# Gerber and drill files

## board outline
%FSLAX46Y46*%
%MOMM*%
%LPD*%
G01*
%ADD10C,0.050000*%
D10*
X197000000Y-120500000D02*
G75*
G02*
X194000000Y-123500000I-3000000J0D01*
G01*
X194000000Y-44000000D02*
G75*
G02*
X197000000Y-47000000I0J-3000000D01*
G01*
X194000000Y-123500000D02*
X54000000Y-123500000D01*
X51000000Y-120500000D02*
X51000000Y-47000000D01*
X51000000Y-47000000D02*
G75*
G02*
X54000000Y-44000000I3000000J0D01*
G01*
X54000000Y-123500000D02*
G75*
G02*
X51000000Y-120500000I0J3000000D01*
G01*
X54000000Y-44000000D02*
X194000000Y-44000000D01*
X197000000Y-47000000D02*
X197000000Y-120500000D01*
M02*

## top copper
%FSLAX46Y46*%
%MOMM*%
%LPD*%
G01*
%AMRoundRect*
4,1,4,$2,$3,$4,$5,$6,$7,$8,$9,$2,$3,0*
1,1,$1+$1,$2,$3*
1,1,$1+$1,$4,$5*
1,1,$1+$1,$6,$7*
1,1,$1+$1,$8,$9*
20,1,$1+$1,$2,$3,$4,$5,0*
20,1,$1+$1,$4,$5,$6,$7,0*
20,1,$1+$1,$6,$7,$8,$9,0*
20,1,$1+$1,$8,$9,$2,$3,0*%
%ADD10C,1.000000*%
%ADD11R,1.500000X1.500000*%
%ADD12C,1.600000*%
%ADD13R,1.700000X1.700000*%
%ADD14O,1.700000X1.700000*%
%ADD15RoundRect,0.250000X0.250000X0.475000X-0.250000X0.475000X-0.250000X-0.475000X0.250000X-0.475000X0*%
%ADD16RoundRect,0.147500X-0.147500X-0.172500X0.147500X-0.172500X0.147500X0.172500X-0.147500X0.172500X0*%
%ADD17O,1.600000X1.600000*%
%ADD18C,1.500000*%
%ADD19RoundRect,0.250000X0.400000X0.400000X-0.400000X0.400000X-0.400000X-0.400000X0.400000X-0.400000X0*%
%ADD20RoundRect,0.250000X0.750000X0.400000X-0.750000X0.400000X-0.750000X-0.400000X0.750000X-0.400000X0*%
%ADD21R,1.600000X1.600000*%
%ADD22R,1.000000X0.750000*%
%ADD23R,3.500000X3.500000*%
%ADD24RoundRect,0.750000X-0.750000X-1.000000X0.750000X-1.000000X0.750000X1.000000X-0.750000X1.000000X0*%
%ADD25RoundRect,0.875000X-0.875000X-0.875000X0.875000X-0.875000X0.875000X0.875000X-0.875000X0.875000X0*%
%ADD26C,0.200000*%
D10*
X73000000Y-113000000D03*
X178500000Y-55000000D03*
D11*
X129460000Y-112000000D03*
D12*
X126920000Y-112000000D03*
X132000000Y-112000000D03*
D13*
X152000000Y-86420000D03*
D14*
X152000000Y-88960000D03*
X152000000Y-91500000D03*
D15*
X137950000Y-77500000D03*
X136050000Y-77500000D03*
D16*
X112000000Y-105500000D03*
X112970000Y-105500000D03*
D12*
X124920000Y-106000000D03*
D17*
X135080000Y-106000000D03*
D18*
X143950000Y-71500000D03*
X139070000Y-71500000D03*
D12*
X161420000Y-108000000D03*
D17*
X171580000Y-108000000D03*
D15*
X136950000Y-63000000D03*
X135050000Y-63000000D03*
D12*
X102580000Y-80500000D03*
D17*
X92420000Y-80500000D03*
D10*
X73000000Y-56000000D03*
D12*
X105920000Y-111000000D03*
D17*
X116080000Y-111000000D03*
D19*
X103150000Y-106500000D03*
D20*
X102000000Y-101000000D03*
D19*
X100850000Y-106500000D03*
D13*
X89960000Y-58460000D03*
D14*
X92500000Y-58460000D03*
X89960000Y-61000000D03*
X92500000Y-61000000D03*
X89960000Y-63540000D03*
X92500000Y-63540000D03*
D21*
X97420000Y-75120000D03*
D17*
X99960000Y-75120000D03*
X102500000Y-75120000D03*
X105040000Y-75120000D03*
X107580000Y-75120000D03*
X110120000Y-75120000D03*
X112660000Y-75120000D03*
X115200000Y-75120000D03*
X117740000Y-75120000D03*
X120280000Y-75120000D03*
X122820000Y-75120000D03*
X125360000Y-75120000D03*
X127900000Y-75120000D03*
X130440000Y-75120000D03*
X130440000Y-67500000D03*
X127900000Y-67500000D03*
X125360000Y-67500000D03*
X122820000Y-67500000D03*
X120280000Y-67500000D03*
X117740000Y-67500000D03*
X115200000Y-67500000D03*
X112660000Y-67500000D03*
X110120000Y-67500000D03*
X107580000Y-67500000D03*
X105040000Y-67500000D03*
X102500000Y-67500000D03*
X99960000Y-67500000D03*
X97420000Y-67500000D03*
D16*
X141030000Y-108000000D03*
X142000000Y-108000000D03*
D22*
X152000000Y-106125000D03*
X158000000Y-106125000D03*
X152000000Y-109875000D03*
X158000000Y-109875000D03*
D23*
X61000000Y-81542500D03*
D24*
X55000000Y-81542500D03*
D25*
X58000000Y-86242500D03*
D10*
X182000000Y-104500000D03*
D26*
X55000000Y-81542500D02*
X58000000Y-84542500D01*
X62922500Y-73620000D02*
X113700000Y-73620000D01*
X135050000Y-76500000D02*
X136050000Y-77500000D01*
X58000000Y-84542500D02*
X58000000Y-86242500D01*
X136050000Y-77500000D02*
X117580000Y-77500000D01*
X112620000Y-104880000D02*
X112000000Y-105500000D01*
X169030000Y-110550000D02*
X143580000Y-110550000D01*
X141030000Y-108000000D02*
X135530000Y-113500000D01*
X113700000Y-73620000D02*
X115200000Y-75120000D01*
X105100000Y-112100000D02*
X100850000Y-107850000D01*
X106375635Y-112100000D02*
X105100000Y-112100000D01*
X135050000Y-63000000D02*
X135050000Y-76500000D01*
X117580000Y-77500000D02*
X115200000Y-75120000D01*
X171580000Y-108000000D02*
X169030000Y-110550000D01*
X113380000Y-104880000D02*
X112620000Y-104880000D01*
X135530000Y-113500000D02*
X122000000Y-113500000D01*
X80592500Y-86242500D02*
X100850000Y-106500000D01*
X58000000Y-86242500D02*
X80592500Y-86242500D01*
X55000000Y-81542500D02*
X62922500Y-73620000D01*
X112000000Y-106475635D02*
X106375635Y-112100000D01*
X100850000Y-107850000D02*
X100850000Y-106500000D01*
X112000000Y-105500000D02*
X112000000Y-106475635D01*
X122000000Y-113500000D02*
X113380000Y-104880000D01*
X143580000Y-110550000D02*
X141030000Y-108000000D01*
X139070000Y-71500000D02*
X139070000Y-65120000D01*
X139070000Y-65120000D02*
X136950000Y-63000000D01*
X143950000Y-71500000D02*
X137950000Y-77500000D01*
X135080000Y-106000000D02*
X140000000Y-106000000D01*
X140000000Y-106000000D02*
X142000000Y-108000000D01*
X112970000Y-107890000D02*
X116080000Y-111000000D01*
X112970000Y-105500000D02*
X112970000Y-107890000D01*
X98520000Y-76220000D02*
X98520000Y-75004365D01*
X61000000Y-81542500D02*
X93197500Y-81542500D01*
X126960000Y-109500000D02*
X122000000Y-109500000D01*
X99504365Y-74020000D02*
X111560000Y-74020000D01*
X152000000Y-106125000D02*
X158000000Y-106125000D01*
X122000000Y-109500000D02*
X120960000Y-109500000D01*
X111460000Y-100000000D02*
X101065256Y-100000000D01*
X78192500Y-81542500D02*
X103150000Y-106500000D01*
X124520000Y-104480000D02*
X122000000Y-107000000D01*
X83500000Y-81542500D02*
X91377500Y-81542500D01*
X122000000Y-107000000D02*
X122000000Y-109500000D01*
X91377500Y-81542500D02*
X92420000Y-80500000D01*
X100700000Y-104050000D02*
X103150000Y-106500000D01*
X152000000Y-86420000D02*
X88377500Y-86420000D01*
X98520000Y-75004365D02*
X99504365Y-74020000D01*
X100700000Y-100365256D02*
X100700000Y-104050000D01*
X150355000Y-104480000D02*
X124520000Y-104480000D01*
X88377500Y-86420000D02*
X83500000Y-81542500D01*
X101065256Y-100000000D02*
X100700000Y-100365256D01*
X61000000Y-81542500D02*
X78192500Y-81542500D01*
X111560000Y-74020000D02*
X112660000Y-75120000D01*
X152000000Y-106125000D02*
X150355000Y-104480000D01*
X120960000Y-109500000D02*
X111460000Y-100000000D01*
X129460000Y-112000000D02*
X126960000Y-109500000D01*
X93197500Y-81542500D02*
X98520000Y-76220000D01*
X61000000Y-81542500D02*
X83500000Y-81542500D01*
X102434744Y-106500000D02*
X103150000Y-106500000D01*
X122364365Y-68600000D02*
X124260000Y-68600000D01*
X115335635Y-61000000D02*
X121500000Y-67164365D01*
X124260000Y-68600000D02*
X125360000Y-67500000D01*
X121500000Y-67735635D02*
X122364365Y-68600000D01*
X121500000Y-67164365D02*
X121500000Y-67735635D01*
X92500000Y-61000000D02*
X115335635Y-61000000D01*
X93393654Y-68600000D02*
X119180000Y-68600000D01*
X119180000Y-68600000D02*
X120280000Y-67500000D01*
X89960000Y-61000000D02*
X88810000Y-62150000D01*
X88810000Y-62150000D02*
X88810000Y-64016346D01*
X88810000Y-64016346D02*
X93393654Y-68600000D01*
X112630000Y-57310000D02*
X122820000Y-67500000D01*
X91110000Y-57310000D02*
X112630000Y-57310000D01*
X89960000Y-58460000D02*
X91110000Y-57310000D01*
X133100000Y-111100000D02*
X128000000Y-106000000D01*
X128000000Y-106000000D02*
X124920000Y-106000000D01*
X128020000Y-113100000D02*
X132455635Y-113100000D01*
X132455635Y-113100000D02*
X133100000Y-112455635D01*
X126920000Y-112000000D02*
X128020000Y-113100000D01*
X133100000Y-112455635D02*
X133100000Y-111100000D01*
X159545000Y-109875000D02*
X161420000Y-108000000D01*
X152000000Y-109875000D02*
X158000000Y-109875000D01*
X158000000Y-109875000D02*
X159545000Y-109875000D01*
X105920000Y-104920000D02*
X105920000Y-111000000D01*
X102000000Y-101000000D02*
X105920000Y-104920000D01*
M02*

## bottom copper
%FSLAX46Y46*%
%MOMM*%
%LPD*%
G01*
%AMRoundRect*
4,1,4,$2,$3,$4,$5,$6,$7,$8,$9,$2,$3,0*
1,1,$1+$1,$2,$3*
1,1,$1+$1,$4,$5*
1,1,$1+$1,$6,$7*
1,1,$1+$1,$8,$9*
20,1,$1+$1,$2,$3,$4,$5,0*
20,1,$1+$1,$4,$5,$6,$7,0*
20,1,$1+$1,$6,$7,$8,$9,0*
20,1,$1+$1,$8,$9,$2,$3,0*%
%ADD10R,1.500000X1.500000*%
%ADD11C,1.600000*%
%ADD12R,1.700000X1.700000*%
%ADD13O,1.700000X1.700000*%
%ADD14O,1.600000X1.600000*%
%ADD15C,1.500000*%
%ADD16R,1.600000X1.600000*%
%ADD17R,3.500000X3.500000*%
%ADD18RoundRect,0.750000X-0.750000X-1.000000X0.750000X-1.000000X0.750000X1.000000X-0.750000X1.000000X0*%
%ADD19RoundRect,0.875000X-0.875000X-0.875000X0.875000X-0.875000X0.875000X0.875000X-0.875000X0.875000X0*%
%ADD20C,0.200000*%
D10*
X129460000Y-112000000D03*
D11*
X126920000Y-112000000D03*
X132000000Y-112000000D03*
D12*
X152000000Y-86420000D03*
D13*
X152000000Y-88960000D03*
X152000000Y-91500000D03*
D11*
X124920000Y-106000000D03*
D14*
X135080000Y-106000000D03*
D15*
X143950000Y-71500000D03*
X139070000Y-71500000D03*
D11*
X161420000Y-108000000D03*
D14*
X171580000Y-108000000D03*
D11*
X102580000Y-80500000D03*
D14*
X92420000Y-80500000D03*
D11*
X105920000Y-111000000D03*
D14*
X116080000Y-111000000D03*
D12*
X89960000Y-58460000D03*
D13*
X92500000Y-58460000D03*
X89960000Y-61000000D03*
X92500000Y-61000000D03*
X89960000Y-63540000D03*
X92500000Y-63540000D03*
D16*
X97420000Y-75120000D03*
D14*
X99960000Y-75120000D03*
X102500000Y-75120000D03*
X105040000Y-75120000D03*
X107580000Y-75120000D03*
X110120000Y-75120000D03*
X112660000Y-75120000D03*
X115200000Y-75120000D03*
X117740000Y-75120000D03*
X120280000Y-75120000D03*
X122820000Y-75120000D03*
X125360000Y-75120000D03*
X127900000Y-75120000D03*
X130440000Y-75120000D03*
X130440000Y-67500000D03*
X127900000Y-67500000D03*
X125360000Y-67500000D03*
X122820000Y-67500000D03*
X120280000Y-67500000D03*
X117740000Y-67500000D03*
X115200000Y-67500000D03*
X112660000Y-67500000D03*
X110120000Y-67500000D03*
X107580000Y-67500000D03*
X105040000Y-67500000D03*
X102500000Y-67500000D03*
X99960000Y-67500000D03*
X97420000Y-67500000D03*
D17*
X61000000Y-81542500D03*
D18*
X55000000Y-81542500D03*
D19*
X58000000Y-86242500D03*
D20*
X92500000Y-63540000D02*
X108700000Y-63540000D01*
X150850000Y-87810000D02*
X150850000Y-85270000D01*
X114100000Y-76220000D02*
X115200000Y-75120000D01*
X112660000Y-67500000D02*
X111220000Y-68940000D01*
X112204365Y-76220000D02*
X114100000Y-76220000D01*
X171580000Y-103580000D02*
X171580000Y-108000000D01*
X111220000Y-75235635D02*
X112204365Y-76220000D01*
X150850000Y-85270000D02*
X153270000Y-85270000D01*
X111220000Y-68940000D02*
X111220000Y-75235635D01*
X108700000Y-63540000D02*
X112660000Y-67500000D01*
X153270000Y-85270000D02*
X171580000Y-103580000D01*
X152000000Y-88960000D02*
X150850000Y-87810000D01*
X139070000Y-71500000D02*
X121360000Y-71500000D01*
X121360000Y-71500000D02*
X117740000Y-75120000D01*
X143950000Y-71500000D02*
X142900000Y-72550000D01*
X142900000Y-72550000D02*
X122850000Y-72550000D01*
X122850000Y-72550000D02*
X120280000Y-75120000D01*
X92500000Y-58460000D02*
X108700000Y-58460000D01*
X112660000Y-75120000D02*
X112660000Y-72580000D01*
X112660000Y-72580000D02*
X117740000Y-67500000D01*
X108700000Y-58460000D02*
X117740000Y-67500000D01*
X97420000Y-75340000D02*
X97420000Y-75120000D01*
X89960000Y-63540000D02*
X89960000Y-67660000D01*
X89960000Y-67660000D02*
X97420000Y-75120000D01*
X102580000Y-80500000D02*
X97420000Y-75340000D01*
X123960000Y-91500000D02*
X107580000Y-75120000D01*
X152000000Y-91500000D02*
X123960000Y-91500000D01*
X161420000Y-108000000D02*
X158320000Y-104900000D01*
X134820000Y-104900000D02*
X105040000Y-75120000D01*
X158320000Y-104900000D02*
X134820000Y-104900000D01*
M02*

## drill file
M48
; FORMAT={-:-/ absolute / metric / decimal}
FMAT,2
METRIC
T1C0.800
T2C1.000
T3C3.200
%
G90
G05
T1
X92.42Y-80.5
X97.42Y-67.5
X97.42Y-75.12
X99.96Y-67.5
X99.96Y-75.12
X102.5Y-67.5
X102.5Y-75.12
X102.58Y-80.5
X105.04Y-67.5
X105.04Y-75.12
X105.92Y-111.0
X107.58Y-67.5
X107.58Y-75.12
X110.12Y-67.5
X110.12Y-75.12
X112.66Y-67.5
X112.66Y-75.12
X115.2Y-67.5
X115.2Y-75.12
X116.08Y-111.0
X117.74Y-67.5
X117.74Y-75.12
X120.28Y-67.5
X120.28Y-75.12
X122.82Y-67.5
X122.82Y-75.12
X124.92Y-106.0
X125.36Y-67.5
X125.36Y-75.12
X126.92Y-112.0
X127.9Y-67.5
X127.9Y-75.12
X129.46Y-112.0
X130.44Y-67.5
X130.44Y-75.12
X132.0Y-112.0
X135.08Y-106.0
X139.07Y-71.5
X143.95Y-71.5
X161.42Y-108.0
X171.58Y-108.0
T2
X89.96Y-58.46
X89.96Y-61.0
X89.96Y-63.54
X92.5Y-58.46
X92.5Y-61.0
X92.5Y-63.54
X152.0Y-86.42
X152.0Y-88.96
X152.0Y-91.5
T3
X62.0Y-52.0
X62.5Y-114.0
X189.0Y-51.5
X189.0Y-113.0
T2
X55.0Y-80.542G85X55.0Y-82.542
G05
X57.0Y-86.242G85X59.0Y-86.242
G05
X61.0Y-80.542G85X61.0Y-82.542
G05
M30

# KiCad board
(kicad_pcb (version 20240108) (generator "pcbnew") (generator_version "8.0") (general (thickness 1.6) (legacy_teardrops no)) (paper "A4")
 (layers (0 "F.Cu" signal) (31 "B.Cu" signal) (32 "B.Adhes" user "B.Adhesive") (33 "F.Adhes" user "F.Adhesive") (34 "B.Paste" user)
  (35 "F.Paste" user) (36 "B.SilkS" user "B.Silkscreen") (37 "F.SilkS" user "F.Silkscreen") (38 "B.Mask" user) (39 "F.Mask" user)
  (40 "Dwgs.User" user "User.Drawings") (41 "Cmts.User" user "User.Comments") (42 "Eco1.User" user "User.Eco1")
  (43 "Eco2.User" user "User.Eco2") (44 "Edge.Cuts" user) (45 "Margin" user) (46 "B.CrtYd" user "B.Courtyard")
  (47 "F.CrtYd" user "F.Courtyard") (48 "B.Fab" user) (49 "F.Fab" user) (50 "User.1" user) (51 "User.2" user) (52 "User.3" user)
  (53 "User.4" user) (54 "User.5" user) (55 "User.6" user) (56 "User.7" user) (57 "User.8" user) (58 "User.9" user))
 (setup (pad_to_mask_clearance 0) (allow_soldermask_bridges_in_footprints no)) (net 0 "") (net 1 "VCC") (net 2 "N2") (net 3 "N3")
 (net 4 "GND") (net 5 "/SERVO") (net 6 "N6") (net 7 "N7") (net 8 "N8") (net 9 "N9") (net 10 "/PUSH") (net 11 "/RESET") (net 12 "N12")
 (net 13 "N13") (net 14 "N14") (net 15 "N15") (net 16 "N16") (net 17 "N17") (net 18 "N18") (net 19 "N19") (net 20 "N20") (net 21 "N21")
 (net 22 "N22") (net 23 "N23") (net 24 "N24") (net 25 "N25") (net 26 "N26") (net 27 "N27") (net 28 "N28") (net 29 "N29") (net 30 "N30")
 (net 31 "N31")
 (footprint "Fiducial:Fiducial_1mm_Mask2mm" (layer "F.Cu") (at 73 113)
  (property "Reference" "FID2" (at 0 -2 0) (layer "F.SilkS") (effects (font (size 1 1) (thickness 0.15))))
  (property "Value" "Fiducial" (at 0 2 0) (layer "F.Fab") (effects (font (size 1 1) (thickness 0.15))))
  (pad "" smd circle (at 0 0) (size 1 1) (layers "F.Cu" "F.Mask") (solder_mask_margin 0.5) (clearance 0.5)))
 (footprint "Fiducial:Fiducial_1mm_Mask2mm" (layer "F.Cu") (at 178.5 55)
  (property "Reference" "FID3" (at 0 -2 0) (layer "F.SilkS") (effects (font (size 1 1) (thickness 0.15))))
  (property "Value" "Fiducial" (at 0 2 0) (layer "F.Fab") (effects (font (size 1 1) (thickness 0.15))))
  (pad "" smd circle (at 0 0) (size 1 1) (layers "F.Cu" "F.Mask") (solder_mask_margin 0.5) (clearance 0.5)))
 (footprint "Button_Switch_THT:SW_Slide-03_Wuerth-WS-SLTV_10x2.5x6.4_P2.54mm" (layer "F.Cu") (at 129.46 112)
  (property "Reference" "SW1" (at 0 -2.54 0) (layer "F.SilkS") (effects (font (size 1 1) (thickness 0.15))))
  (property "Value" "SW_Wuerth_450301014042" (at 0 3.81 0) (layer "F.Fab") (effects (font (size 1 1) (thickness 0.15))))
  (pad "1" thru_hole rect (at 0 0) (size 1.5 1.5) (drill 0.8) (layers "*.Cu" "*.Mask") (remove_unused_layers no) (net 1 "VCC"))
  (pad "2" thru_hole circle (at -2.54 0) (size 1.6 1.6) (drill 0.8) (layers "*.Cu" "*.Mask") (remove_unused_layers no) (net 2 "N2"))
  (pad "3" thru_hole circle (at 2.54 0) (size 1.6 1.6) (drill 0.8) (layers "*.Cu" "*.Mask") (remove_unused_layers no) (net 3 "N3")))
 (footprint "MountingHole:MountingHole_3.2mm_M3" (layer "F.Cu") (at 62.5 114)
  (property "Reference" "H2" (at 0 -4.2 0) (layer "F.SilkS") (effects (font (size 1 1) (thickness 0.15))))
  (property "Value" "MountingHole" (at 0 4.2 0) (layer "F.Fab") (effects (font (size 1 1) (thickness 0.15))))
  (pad "" np_thru_hole circle (at 0 0) (size 3.2 3.2) (drill 3.2) (layers "*.Cu" "*.Mask")))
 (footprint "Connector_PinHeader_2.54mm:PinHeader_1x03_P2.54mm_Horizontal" (layer "F.Cu") (at 152 86.42)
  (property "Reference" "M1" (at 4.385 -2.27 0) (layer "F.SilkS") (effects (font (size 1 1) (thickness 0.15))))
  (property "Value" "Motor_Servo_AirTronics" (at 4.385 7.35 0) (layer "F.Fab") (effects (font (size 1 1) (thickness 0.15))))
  (pad "1" thru_hole rect (at 0 0) (size 1.7 1.7) (drill 1) (layers "*.Cu" "*.Mask") (remove_unused_layers no) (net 1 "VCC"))
  (pad "2" thru_hole oval (at 0 2.54) (size 1.7 1.7) (drill 1) (layers "*.Cu" "*.Mask") (remove_unused_layers no) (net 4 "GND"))
  (pad "3" thru_hole oval (at 0 5.08) (size 1.7 1.7) (drill 1) (layers "*.Cu" "*.Mask") (remove_unused_layers no) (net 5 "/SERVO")))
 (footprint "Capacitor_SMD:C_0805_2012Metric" (layer "F.Cu") (at 137 77.5 180)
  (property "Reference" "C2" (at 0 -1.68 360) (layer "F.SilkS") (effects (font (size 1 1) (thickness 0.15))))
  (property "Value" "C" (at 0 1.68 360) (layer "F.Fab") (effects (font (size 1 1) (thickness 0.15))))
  (pad "1" smd roundrect (at -0.95 0 180) (size 1 1.45) (layers "F.Cu" "F.Paste" "F.Mask") (roundrect_rratio 0.25) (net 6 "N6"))
  (pad "2" smd roundrect (at 0.95 0 180) (size 1 1.45) (layers "F.Cu" "F.Paste" "F.Mask") (roundrect_rratio 0.25) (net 4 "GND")))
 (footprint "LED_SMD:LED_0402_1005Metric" (layer "F.Cu") (at 112.485 105.5)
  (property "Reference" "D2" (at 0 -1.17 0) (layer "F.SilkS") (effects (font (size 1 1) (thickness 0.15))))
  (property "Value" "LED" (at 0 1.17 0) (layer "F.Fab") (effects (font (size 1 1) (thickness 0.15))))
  (pad "1" smd roundrect (at -0.485 0) (size 0.59 0.64) (layers "F.Cu" "F.Paste" "F.Mask") (roundrect_rratio 0.25) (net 4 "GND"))
  (pad "2" smd roundrect (at 0.485 0) (size 0.59 0.64) (layers "F.Cu" "F.Paste" "F.Mask") (roundrect_rratio 0.25) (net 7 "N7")))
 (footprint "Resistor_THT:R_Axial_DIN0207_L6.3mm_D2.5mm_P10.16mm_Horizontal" (layer "F.Cu") (at 124.92 106)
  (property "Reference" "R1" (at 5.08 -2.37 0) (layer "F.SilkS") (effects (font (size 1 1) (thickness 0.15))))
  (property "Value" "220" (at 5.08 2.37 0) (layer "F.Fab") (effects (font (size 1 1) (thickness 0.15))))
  (pad "1" thru_hole circle (at 0 0) (size 1.6 1.6) (drill 0.8) (layers "*.Cu" "*.Mask") (remove_unused_layers no) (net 2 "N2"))
  (pad "2" thru_hole oval (at 10.16 0) (size 1.6 1.6) (drill 0.8) (layers "*.Cu" "*.Mask") (remove_unused_layers no) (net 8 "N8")))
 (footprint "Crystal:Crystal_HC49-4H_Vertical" (layer "F.Cu") (at 143.95 71.5 180)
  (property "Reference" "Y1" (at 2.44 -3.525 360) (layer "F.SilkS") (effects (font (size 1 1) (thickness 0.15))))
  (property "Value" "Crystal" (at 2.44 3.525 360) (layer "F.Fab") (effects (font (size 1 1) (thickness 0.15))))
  (pad "1" thru_hole circle (at 0 0 180) (size 1.5 1.5) (drill 0.8) (layers "*.Cu" "*.Mask") (remove_unused_layers no) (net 6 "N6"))
  (pad "2" thru_hole circle (at 4.88 0 180) (size 1.5 1.5) (drill 0.8) (layers "*.Cu" "*.Mask") (remove_unused_layers no) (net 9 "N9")))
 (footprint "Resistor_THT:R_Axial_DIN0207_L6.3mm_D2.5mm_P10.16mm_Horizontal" (layer "F.Cu") (at 161.42 108)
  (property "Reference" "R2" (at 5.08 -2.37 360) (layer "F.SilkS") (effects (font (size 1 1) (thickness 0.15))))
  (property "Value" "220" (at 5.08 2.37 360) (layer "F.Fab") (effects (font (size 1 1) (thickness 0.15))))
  (pad "1" thru_hole circle (at 0 0) (size 1.6 1.6) (drill 0.8) (layers "*.Cu" "*.Mask") (remove_unused_layers no) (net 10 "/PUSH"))
  (pad "2" thru_hole oval (at 10.16 0) (size 1.6 1.6) (drill 0.8) (layers "*.Cu" "*.Mask") (remove_unused_layers no) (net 4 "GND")))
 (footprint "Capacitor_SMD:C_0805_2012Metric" (layer "F.Cu") (at 136 63 180)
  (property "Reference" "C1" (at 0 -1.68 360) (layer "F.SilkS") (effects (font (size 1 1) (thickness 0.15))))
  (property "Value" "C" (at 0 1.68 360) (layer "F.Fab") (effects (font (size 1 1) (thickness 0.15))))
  (pad "1" smd roundrect (at -0.95 0 180) (size 1 1.45) (layers "F.Cu" "F.Paste" "F.Mask") (roundrect_rratio 0.25) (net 9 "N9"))
  (pad "2" smd roundrect (at 0.95 0 180) (size 1 1.45) (layers "F.Cu" "F.Paste" "F.Mask") (roundrect_rratio 0.25) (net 4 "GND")))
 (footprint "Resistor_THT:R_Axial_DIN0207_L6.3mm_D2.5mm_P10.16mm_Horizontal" (layer "F.Cu") (at 102.58 80.5 180)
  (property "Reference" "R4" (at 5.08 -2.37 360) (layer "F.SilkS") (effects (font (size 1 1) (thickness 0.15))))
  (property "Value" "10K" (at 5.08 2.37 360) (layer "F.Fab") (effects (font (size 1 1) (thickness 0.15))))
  (pad "1" thru_hole circle (at 0 0 180) (size 1.6 1.6) (drill 0.8) (layers "*.Cu" "*.Mask") (remove_unused_layers no) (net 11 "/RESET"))
  (pad "2" thru_hole oval (at 10.16 0 180) (size 1.6 1.6) (drill 0.8) (layers "*.Cu" "*.Mask") (remove_unused_layers no) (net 1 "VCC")))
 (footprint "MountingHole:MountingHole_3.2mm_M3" (layer "F.Cu") (at 189 51.5)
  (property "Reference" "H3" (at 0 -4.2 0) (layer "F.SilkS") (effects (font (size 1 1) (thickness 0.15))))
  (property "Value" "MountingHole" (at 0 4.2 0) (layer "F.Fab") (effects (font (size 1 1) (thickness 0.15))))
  (pad "" np_thru_hole circle (at 0 0) (size 3.2 3.2) (drill 3.2) (layers "*.Cu" "*.Mask")))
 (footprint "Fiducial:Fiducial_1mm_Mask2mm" (layer "F.Cu") (at 73 56)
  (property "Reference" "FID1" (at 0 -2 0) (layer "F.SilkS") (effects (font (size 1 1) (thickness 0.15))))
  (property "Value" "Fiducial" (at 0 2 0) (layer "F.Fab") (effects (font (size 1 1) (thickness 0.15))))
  (pad "" smd circle (at 0 0) (size 1 1) (layers "F.Cu" "F.Mask") (solder_mask_margin 0.5) (clearance 0.5)))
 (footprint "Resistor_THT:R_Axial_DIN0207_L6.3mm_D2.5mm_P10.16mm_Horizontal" (layer "F.Cu") (at 105.92 111)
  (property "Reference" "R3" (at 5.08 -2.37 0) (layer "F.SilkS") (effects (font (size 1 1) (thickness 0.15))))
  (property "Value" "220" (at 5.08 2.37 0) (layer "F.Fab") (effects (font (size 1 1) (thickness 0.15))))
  (pad "1" thru_hole circle (at 0 0) (size 1.6 1.6) (drill 0.8) (layers "*.Cu" "*.Mask") (remove_unused_layers no) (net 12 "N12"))
  (pad "2" thru_hole oval (at 10.16 0) (size 1.6 1.6) (drill 0.8) (layers "*.Cu" "*.Mask") (remove_unused_layers no) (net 7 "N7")))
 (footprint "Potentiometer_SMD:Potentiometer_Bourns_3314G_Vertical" (layer "F.Cu") (at 102 103.75 180)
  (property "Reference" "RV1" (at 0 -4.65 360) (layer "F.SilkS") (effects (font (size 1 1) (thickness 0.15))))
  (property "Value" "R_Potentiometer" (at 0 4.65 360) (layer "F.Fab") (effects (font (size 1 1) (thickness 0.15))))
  (pad "1" smd roundrect (at -1.15 -2.75 180) (size 1.3 1.3) (layers "F.Cu" "F.Paste" "F.Mask") (roundrect_rratio 0.1923076923)
   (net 1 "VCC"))
  (pad "2" smd roundrect (at 0 2.75 180) (size 2 1.3) (layers "F.Cu" "F.Paste" "F.Mask") (roundrect_rratio 0.1923076923) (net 12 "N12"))
  (pad "3" smd roundrect (at 1.15 -2.75 180) (size 1.3 1.3) (layers "F.Cu" "F.Paste" "F.Mask") (roundrect_rratio 0.1923076923) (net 4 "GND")))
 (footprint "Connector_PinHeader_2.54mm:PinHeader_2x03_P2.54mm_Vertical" (layer "F.Cu") (at 89.96 58.46)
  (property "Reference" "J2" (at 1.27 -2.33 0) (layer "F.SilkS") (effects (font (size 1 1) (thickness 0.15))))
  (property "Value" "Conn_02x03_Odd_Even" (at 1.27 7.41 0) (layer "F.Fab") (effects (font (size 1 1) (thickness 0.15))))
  (pad "1" thru_hole rect (at 0 0) (size 1.7 1.7) (drill 1) (layers "*.Cu" "*.Mask") (remove_unused_layers no) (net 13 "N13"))
  (pad "2" thru_hole oval (at 2.54 0) (size 1.7 1.7) (drill 1) (layers "*.Cu" "*.Mask") (remove_unused_layers no) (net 1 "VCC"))
  (pad "3" thru_hole oval (at 0 2.54) (size 1.7 1.7) (drill 1) (layers "*.Cu" "*.Mask") (remove_unused_layers no) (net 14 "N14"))
  (pad "4" thru_hole oval (at 2.54 2.54) (size 1.7 1.7) (drill 1) (layers "*.Cu" "*.Mask") (remove_unused_layers no) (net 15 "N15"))
  (pad "5" thru_hole oval (at 0 5.08) (size 1.7 1.7) (drill 1) (layers "*.Cu" "*.Mask") (remove_unused_layers no) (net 11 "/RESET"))
  (pad "6" thru_hole oval (at 2.54 5.08) (size 1.7 1.7) (drill 1) (layers "*.Cu" "*.Mask") (remove_unused_layers no) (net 4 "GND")))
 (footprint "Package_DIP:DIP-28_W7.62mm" (layer "F.Cu") (at 97.42 75.12 90)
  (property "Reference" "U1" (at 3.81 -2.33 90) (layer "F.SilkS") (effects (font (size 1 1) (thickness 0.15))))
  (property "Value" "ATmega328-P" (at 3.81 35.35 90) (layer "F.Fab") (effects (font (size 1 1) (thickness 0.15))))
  (pad "1" thru_hole rect (at 0 0 90) (size 1.6 1.6) (drill 0.8) (layers "*.Cu" "*.Mask") (remove_unused_layers no) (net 11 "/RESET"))
  (pad "2" thru_hole oval (at 0 2.54 90) (size 1.6 1.6) (drill 0.8) (layers "*.Cu" "*.Mask") (remove_unused_layers no) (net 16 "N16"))
  (pad "3" thru_hole oval (at 0 5.08 90) (size 1.6 1.6) (drill 0.8) (layers "*.Cu" "*.Mask") (remove_unused_layers no) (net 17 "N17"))
  (pad "4" thru_hole oval (at 0 7.62 90) (size 1.6 1.6) (drill 0.8) (layers "*.Cu" "*.Mask") (remove_unused_layers no) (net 10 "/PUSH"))
  (pad "5" thru_hole oval (at 0 10.16 90) (size 1.6 1.6) (drill 0.8) (layers "*.Cu" "*.Mask") (remove_unused_layers no) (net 5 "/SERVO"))
  (pad "6" thru_hole oval (at 0 12.7 90) (size 1.6 1.6) (drill 0.8) (layers "*.Cu" "*.Mask") (remove_unused_layers no) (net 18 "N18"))
  (pad "7" thru_hole oval (at 0 15.24 90) (size 1.6 1.6) (drill 0.8) (layers "*.Cu" "*.Mask") (remove_unused_layers no) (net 1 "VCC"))
  (pad "8" thru_hole oval (at 0 17.78 90) (size 1.6 1.6) (drill 0.8) (layers "*.Cu" "*.Mask") (remove_unused_layers no) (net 4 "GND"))
  (pad "9" thru_hole oval (at 0 20.32 90) (size 1.6 1.6) (drill 0.8) (layers "*.Cu" "*.Mask") (remove_unused_layers no) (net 9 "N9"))
  (pad "10" thru_hole oval (at 0 22.86 90) (size 1.6 1.6) (drill 0.8) (layers "*.Cu" "*.Mask") (remove_unused_layers no) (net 6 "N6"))
  (pad "11" thru_hole oval (at 0 25.4 90) (size 1.6 1.6) (drill 0.8) (layers "*.Cu" "*.Mask") (remove_unused_layers no) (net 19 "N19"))
  (pad "12" thru_hole oval (at 0 27.94 90) (size 1.6 1.6) (drill 0.8) (layers "*.Cu" "*.Mask") (remove_unused_layers no) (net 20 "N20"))
  (pad "13" thru_hole oval (at 0 30.48 90) (size 1.6 1.6) (drill 0.8) (layers "*.Cu" "*.Mask") (remove_unused_layers no) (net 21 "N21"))
  (pad "14" thru_hole oval (at 0 33.02 90) (size 1.6 1.6) (drill 0.8) (layers "*.Cu" "*.Mask") (remove_unused_layers no) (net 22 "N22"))
  (pad "15" thru_hole oval (at 7.62 33.02 90) (size 1.6 1.6) (drill 0.8) (layers "*.Cu" "*.Mask") (remove_unused_layers no) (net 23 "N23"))
  (pad "16" thru_hole oval (at 7.62 30.48 90) (size 1.6 1.6) (drill 0.8) (layers "*.Cu" "*.Mask") (remove_unused_layers no) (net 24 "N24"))
  (pad "17" thru_hole oval (at 7.62 27.94 90) (size 1.6 1.6) (drill 0.8) (layers "*.Cu" "*.Mask") (remove_unused_layers no) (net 15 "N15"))
  (pad "18" thru_hole oval (at 7.62 25.4 90) (size 1.6 1.6) (drill 0.8) (layers "*.Cu" "*.Mask") (remove_unused_layers no) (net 13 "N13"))
  (pad "19" thru_hole oval (at 7.62 22.86 90) (size 1.6 1.6) (drill 0.8) (layers "*.Cu" "*.Mask") (remove_unused_layers no) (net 14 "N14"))
  (pad "20" thru_hole oval (at 7.62 20.32 90) (size 1.6 1.6) (drill 0.8) (layers "*.Cu" "*.Mask") (remove_unused_layers no) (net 1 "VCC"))
  (pad "21" thru_hole oval (at 7.62 17.78 90) (size 1.6 1.6) (drill 0.8) (layers "*.Cu" "*.Mask") (remove_unused_layers no) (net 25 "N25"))
  (pad "22" thru_hole oval (at 7.62 15.24 90) (size 1.6 1.6) (drill 0.8) (layers "*.Cu" "*.Mask") (remove_unused_layers no) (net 4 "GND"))
  (pad "23" thru_hole oval (at 7.62 12.7 90) (size 1.6 1.6) (drill 0.8) (layers "*.Cu" "*.Mask") (remove_unused_layers no) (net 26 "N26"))
  (pad "24" thru_hole oval (at 7.62 10.16 90) (size 1.6 1.6) (drill 0.8) (layers "*.Cu" "*.Mask") (remove_unused_layers no) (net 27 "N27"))
  (pad "25" thru_hole oval (at 7.62 7.62 90) (size 1.6 1.6) (drill 0.8) (layers "*.Cu" "*.Mask") (remove_unused_layers no) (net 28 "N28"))
  (pad "26" thru_hole oval (at 7.62 5.08 90) (size 1.6 1.6) (drill 0.8) (layers "*.Cu" "*.Mask") (remove_unused_layers no) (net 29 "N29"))
  (pad "27" thru_hole oval (at 7.62 2.54 90) (size 1.6 1.6) (drill 0.8) (layers "*.Cu" "*.Mask") (remove_unused_layers no) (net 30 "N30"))
  (pad "28" thru_hole oval (at 7.62 0 90) (size 1.6 1.6) (drill 0.8) (layers "*.Cu" "*.Mask") (remove_unused_layers no) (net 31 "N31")))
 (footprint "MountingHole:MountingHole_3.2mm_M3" (layer "F.Cu") (at 189 113)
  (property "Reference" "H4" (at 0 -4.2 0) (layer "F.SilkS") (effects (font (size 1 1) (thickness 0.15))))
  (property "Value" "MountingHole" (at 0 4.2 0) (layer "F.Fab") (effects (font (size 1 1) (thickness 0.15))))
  (pad "" np_thru_hole circle (at 0 0) (size 3.2 3.2) (drill 3.2) (layers "*.Cu" "*.Mask")))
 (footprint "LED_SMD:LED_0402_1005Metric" (layer "F.Cu") (at 141.515 108)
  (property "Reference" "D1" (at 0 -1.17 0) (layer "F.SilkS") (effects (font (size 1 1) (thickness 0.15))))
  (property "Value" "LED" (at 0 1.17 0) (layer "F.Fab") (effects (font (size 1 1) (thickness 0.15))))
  (pad "1" smd roundrect (at -0.485 0) (size 0.59 0.64) (layers "F.Cu" "F.Paste" "F.Mask") (roundrect_rratio 0.25) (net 4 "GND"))
  (pad "2" smd roundrect (at 0.485 0) (size 0.59 0.64) (layers "F.Cu" "F.Paste" "F.Mask") (roundrect_rratio 0.25) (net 8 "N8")))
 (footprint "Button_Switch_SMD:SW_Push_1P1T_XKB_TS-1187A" (layer "F.Cu") (at 155 108)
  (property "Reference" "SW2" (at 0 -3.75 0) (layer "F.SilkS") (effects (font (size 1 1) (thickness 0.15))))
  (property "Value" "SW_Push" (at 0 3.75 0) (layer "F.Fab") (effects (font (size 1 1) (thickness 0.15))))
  (pad "1" smd rect (at -3 -1.875) (size 1 0.75) (layers "F.Cu" "F.Paste" "F.Mask") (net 1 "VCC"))
  (pad "1" smd rect (at 3 -1.875) (size 1 0.75) (layers "F.Cu" "F.Paste" "F.Mask") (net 1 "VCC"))
  (pad "2" smd rect (at -3 1.875) (size 1 0.75) (layers "F.Cu" "F.Paste" "F.Mask") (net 10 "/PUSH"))
  (pad "2" smd rect (at 3 1.875) (size 1 0.75) (layers "F.Cu" "F.Paste" "F.Mask") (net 10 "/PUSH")))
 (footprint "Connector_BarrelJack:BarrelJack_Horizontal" (layer "F.Cu") (at 61 81.5425)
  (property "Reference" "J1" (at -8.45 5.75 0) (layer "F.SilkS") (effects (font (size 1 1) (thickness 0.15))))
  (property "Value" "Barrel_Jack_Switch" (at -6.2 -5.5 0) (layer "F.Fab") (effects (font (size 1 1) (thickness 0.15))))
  (pad "1" thru_hole rect (at 0 0) (size 3.5 3.5) (drill oval 1 3) (layers "*.Cu" "*.Mask") (remove_unused_layers no) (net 1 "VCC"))
  (pad "2" thru_hole roundrect (at -6 0) (size 3 3.5) (drill oval 1 3) (layers "*.Cu" "*.Mask") (remove_unused_layers no)
   (roundrect_rratio 0.25) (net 4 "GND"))
  (pad "3" thru_hole roundrect (at -3 4.7) (size 3.5 3.5) (drill oval 3 1) (layers "*.Cu" "*.Mask") (remove_unused_layers no)
   (roundrect_rratio 0.25) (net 4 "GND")))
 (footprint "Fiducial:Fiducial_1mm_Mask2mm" (layer "F.Cu") (at 182 104.5)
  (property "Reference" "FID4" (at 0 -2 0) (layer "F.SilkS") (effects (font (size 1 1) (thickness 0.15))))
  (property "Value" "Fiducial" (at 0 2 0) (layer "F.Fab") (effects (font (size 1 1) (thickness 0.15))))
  (pad "" smd circle (at 0 0) (size 1 1) (layers "F.Cu" "F.Mask") (solder_mask_margin 0.5) (clearance 0.5)))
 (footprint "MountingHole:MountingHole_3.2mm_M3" (layer "F.Cu") (at 62 52)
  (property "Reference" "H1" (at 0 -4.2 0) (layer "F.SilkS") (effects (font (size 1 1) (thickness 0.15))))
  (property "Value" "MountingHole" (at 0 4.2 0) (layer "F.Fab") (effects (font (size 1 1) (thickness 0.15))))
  (pad "" np_thru_hole circle (at 0 0) (size 3.2 3.2) (drill 3.2) (layers "*.Cu" "*.Mask")))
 (gr_arc (start 197 120.5) (mid 196.12132 122.62132) (end 194 123.5) (stroke (width 0.05) (type default)) (layer "Edge.Cuts"))
 (gr_arc (start 194 44) (mid 196.12132 44.87868) (end 197 47) (stroke (width 0.05) (type default)) (layer "Edge.Cuts"))
 (gr_line (start 194 123.5) (end 54 123.5) (stroke (width 0.05) (type default)) (layer "Edge.Cuts"))
 (gr_line (start 51 120.5) (end 51 47) (stroke (width 0.05) (type default)) (layer "Edge.Cuts"))
 (gr_arc (start 51 47) (mid 51.87868 44.87868) (end 54 44) (stroke (width 0.05) (type default)) (layer "Edge.Cuts"))
 (gr_arc (start 54 123.5) (mid 51.87868 122.62132) (end 51 120.5) (stroke (width 0.05) (type default)) (layer "Edge.Cuts"))
 (gr_line (start 54 44) (end 194 44) (stroke (width 0.05) (type default)) (layer "Edge.Cuts"))
 (gr_line (start 197 47) (end 197 120.5) (stroke (width 0.05) (type default)) (layer "Edge.Cuts"))
 (segment (start 55 81.5425) (end 58 84.5425) (width 0.2) (layer "F.Cu") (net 4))
 (segment (start 62.9225 73.62) (end 113.7 73.62) (width 0.2) (layer "F.Cu") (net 4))
 (segment (start 135.05 76.5) (end 136.05 77.5) (width 0.2) (layer "F.Cu") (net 4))
 (segment (start 58 84.5425) (end 58 86.2425) (width 0.2) (layer "F.Cu") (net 4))
 (segment (start 136.05 77.5) (end 117.58 77.5) (width 0.2) (layer "F.Cu") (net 4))
 (segment (start 112.62 104.88) (end 112 105.5) (width 0.2) (layer "F.Cu") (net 4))
 (segment (start 169.03 110.55) (end 143.58 110.55) (width 0.2) (layer "F.Cu") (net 4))
 (segment (start 141.03 108) (end 135.53 113.5) (width 0.2) (layer "F.Cu") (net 4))
 (segment (start 113.7 73.62) (end 115.2 75.12) (width 0.2) (layer "F.Cu") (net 4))
 (segment (start 105.1 112.1) (end 100.85 107.85) (width 0.2) (layer "F.Cu") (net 4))
 (segment (start 106.375635 112.1) (end 105.1 112.1) (width 0.2) (layer "F.Cu") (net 4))
 (segment (start 135.05 63) (end 135.05 76.5) (width 0.2) (layer "F.Cu") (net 4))
 (segment (start 117.58 77.5) (end 115.2 75.12) (width 0.2) (layer "F.Cu") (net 4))
 (segment (start 171.58 108) (end 169.03 110.55) (width 0.2) (layer "F.Cu") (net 4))
 (segment (start 113.38 104.88) (end 112.62 104.88) (width 0.2) (layer "F.Cu") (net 4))
 (segment (start 135.53 113.5) (end 122 113.5) (width 0.2) (layer "F.Cu") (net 4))
 (segment (start 80.5925 86.2425) (end 100.85 106.5) (width 0.2) (layer "F.Cu") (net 4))
 (segment (start 58 86.2425) (end 80.5925 86.2425) (width 0.2) (layer "F.Cu") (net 4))
 (segment (start 55 81.5425) (end 62.9225 73.62) (width 0.2) (layer "F.Cu") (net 4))
 (segment (start 112 106.475635) (end 106.375635 112.1) (width 0.2) (layer "F.Cu") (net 4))
 (segment (start 100.85 107.85) (end 100.85 106.5) (width 0.2) (layer "F.Cu") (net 4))
 (segment (start 112 105.5) (end 112 106.475635) (width 0.2) (layer "F.Cu") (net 4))
 (segment (start 122 113.5) (end 113.38 104.88) (width 0.2) (layer "F.Cu") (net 4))
 (segment (start 143.58 110.55) (end 141.03 108) (width 0.2) (layer "F.Cu") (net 4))
 (segment (start 92.5 63.54) (end 108.7 63.54) (width 0.2) (layer "B.Cu") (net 4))
 (segment (start 150.85 87.81) (end 150.85 85.27) (width 0.2) (layer "B.Cu") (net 4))
 (segment (start 114.1 76.22) (end 115.2 75.12) (width 0.2) (layer "B.Cu") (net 4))
 (segment (start 112.66 67.5) (end 111.22 68.94) (width 0.2) (layer "B.Cu") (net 4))
 (segment (start 112.204365 76.22) (end 114.1 76.22) (width 0.2) (layer "B.Cu") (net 4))
 (segment (start 171.58 103.58) (end 171.58 108) (width 0.2) (layer "B.Cu") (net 4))
 (segment (start 111.22 75.235635) (end 112.204365 76.22) (width 0.2) (layer "B.Cu") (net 4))
 (segment (start 150.85 85.27) (end 153.27 85.27) (width 0.2) (layer "B.Cu") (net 4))
 (segment (start 111.22 68.94) (end 111.22 75.235635) (width 0.2) (layer "B.Cu") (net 4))
 (segment (start 108.7 63.54) (end 112.66 67.5) (width 0.2) (layer "B.Cu") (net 4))
 (segment (start 153.27 85.27) (end 171.58 103.58) (width 0.2) (layer "B.Cu") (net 4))
 (segment (start 152 88.96) (end 150.85 87.81) (width 0.2) (layer "B.Cu") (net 4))
 (segment (start 139.07 71.5) (end 139.07 65.12) (width 0.2) (layer "F.Cu") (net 9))
 (segment (start 139.07 65.12) (end 136.95 63) (width 0.2) (layer "F.Cu") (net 9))
 (segment (start 139.07 71.5) (end 121.36 71.5) (width 0.2) (layer "B.Cu") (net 9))
 (segment (start 121.36 71.5) (end 117.74 75.12) (width 0.2) (layer "B.Cu") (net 9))
 (segment (start 143.95 71.5) (end 137.95 77.5) (width 0.2) (layer "F.Cu") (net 6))
 (segment (start 143.95 71.5) (end 142.9 72.55) (width 0.2) (layer "B.Cu") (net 6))
 (segment (start 142.9 72.55) (end 122.85 72.55) (width 0.2) (layer "B.Cu") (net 6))
 (segment (start 122.85 72.55) (end 120.28 75.12) (width 0.2) (layer "B.Cu") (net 6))
 (segment (start 135.08 106) (end 140 106) (width 0.2) (layer "F.Cu") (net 8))
 (segment (start 140 106) (end 142 108) (width 0.2) (layer "F.Cu") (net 8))
 (segment (start 112.97 107.89) (end 116.08 111) (width 0.2) (layer "F.Cu") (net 7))
 (segment (start 112.97 105.5) (end 112.97 107.89) (width 0.2) (layer "F.Cu") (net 7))
 (segment (start 98.52 76.22) (end 98.52 75.004365) (width 0.2) (layer "F.Cu") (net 1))
 (segment (start 61 81.5425) (end 93.1975 81.5425) (width 0.2) (layer "F.Cu") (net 1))
 (segment (start 126.96 109.5) (end 122 109.5) (width 0.2) (layer "F.Cu") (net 1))
 (segment (start 99.504365 74.02) (end 111.56 74.02) (width 0.2) (layer "F.Cu") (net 1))
 (segment (start 152 106.125) (end 158 106.125) (width 0.2) (layer "F.Cu") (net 1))
 (segment (start 122 109.5) (end 120.96 109.5) (width 0.2) (layer "F.Cu") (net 1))
 (segment (start 111.46 100) (end 101.065256 100) (width 0.2) (layer "F.Cu") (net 1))
 (segment (start 78.1925 81.5425) (end 103.15 106.5) (width 0.2) (layer "F.Cu") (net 1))
 (segment (start 124.52 104.48) (end 122 107) (width 0.2) (layer "F.Cu") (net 1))
 (segment (start 83.5 81.5425) (end 91.3775 81.5425) (width 0.2) (layer "F.Cu") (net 1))
 (segment (start 122 107) (end 122 109.5) (width 0.2) (layer "F.Cu") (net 1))
 (segment (start 91.3775 81.5425) (end 92.42 80.5) (width 0.2) (layer "F.Cu") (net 1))
 (segment (start 100.7 104.05) (end 103.15 106.5) (width 0.2) (layer "F.Cu") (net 1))
 (segment (start 152 86.42) (end 88.3775 86.42) (width 0.2) (layer "F.Cu") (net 1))
 (segment (start 98.52 75.004365) (end 99.504365 74.02) (width 0.2) (layer "F.Cu") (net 1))
 (segment (start 100.7 100.365256) (end 100.7 104.05) (width 0.2) (layer "F.Cu") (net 1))
 (segment (start 150.355 104.48) (end 124.52 104.48) (width 0.2) (layer "F.Cu") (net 1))
 (segment (start 88.3775 86.42) (end 83.5 81.5425) (width 0.2) (layer "F.Cu") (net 1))
 (segment (start 101.065256 100) (end 100.7 100.365256) (width 0.2) (layer "F.Cu") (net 1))
 (segment (start 61 81.5425) (end 78.1925 81.5425) (width 0.2) (layer "F.Cu") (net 1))
 (segment (start 111.56 74.02) (end 112.66 75.12) (width 0.2) (layer "F.Cu") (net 1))
 (segment (start 152 106.125) (end 150.355 104.48) (width 0.2) (layer "F.Cu") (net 1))
 (segment (start 120.96 109.5) (end 111.46 100) (width 0.2) (layer "F.Cu") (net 1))
 (segment (start 129.46 112) (end 126.96 109.5) (width 0.2) (layer "F.Cu") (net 1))
 (segment (start 93.1975 81.5425) (end 98.52 76.22) (width 0.2) (layer "F.Cu") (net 1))
 (segment (start 61 81.5425) (end 83.5 81.5425) (width 0.2) (layer "F.Cu") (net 1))
 (segment (start 102.434744 106.5) (end 103.15 106.5) (width 0.2) (layer "F.Cu") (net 1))
 (segment (start 92.5 58.46) (end 108.7 58.46) (width 0.2) (layer "B.Cu") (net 1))
 (segment (start 112.66 75.12) (end 112.66 72.58) (width 0.2) (layer "B.Cu") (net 1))
 (segment (start 112.66 72.58) (end 117.74 67.5) (width 0.2) (layer "B.Cu") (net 1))
 (segment (start 108.7 58.46) (end 117.74 67.5) (width 0.2) (layer "B.Cu") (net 1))
 (segment (start 122.364365 68.6) (end 124.26 68.6) (width 0.2) (layer "F.Cu") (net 15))
 (segment (start 115.335635 61) (end 121.5 67.164365) (width 0.2) (layer "F.Cu") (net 15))
 (segment (start 124.26 68.6) (end 125.36 67.5) (width 0.2) (layer "F.Cu") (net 15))
 (segment (start 121.5 67.735635) (end 122.364365 68.6) (width 0.2) (layer "F.Cu") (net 15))
 (segment (start 121.5 67.164365) (end 121.5 67.735635) (width 0.2) (layer "F.Cu") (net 15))
 (segment (start 92.5 61) (end 115.335635 61) (width 0.2) (layer "F.Cu") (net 15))
 (segment (start 93.393654 68.6) (end 119.18 68.6) (width 0.2) (layer "F.Cu") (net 14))
 (segment (start 119.18 68.6) (end 120.28 67.5) (width 0.2) (layer "F.Cu") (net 14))
 (segment (start 89.96 61) (end 88.81 62.15) (width 0.2) (layer "F.Cu") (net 14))
 (segment (start 88.81 62.15) (end 88.81 64.016346) (width 0.2) (layer "F.Cu") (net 14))
 (segment (start 88.81 64.016346) (end 93.393654 68.6) (width 0.2) (layer "F.Cu") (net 14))
 (segment (start 97.42 75.34) (end 97.42 75.12) (width 0.2) (layer "B.Cu") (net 11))
 (segment (start 89.96 63.54) (end 89.96 67.66) (width 0.2) (layer "B.Cu") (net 11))
 (segment (start 89.96 67.66) (end 97.42 75.12) (width 0.2) (layer "B.Cu") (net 11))
 (segment (start 102.58 80.5) (end 97.42 75.34) (width 0.2) (layer "B.Cu") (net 11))
 (segment (start 112.63 57.31) (end 122.82 67.5) (width 0.2) (layer "F.Cu") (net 13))
 (segment (start 91.11 57.31) (end 112.63 57.31) (width 0.2) (layer "F.Cu") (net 13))
 (segment (start 89.96 58.46) (end 91.11 57.31) (width 0.2) (layer "F.Cu") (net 13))
 (segment (start 123.96 91.5) (end 107.58 75.12) (width 0.2) (layer "B.Cu") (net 5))
 (segment (start 152 91.5) (end 123.96 91.5) (width 0.2) (layer "B.Cu") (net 5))
 (segment (start 133.1 111.1) (end 128 106) (width 0.2) (layer "F.Cu") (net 2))
 (segment (start 128 106) (end 124.92 106) (width 0.2) (layer "F.Cu") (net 2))
 (segment (start 128.02 113.1) (end 132.455635 113.1) (width 0.2) (layer "F.Cu") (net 2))
 (segment (start 132.455635 113.1) (end 133.1 112.455635) (width 0.2) (layer "F.Cu") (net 2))
 (segment (start 126.92 112) (end 128.02 113.1) (width 0.2) (layer "F.Cu") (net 2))
 (segment (start 133.1 112.455635) (end 133.1 111.1) (width 0.2) (layer "F.Cu") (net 2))
 (segment (start 159.545 109.875) (end 161.42 108) (width 0.2) (layer "F.Cu") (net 10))
 (segment (start 152 109.875) (end 158 109.875) (width 0.2) (layer "F.Cu") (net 10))
 (segment (start 158 109.875) (end 159.545 109.875) (width 0.2) (layer "F.Cu") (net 10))
 (segment (start 161.42 108) (end 158.32 104.9) (width 0.2) (layer "B.Cu") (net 10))
 (segment (start 134.82 104.9) (end 105.04 75.12) (width 0.2) (layer "B.Cu") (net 10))
 (segment (start 158.32 104.9) (end 134.82 104.9) (width 0.2) (layer "B.Cu") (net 10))
 (segment (start 105.92 104.92) (end 105.92 111) (width 0.2) (layer "F.Cu") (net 12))
 (segment (start 102 101) (end 105.92 104.92) (width 0.2) (layer "F.Cu") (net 12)))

